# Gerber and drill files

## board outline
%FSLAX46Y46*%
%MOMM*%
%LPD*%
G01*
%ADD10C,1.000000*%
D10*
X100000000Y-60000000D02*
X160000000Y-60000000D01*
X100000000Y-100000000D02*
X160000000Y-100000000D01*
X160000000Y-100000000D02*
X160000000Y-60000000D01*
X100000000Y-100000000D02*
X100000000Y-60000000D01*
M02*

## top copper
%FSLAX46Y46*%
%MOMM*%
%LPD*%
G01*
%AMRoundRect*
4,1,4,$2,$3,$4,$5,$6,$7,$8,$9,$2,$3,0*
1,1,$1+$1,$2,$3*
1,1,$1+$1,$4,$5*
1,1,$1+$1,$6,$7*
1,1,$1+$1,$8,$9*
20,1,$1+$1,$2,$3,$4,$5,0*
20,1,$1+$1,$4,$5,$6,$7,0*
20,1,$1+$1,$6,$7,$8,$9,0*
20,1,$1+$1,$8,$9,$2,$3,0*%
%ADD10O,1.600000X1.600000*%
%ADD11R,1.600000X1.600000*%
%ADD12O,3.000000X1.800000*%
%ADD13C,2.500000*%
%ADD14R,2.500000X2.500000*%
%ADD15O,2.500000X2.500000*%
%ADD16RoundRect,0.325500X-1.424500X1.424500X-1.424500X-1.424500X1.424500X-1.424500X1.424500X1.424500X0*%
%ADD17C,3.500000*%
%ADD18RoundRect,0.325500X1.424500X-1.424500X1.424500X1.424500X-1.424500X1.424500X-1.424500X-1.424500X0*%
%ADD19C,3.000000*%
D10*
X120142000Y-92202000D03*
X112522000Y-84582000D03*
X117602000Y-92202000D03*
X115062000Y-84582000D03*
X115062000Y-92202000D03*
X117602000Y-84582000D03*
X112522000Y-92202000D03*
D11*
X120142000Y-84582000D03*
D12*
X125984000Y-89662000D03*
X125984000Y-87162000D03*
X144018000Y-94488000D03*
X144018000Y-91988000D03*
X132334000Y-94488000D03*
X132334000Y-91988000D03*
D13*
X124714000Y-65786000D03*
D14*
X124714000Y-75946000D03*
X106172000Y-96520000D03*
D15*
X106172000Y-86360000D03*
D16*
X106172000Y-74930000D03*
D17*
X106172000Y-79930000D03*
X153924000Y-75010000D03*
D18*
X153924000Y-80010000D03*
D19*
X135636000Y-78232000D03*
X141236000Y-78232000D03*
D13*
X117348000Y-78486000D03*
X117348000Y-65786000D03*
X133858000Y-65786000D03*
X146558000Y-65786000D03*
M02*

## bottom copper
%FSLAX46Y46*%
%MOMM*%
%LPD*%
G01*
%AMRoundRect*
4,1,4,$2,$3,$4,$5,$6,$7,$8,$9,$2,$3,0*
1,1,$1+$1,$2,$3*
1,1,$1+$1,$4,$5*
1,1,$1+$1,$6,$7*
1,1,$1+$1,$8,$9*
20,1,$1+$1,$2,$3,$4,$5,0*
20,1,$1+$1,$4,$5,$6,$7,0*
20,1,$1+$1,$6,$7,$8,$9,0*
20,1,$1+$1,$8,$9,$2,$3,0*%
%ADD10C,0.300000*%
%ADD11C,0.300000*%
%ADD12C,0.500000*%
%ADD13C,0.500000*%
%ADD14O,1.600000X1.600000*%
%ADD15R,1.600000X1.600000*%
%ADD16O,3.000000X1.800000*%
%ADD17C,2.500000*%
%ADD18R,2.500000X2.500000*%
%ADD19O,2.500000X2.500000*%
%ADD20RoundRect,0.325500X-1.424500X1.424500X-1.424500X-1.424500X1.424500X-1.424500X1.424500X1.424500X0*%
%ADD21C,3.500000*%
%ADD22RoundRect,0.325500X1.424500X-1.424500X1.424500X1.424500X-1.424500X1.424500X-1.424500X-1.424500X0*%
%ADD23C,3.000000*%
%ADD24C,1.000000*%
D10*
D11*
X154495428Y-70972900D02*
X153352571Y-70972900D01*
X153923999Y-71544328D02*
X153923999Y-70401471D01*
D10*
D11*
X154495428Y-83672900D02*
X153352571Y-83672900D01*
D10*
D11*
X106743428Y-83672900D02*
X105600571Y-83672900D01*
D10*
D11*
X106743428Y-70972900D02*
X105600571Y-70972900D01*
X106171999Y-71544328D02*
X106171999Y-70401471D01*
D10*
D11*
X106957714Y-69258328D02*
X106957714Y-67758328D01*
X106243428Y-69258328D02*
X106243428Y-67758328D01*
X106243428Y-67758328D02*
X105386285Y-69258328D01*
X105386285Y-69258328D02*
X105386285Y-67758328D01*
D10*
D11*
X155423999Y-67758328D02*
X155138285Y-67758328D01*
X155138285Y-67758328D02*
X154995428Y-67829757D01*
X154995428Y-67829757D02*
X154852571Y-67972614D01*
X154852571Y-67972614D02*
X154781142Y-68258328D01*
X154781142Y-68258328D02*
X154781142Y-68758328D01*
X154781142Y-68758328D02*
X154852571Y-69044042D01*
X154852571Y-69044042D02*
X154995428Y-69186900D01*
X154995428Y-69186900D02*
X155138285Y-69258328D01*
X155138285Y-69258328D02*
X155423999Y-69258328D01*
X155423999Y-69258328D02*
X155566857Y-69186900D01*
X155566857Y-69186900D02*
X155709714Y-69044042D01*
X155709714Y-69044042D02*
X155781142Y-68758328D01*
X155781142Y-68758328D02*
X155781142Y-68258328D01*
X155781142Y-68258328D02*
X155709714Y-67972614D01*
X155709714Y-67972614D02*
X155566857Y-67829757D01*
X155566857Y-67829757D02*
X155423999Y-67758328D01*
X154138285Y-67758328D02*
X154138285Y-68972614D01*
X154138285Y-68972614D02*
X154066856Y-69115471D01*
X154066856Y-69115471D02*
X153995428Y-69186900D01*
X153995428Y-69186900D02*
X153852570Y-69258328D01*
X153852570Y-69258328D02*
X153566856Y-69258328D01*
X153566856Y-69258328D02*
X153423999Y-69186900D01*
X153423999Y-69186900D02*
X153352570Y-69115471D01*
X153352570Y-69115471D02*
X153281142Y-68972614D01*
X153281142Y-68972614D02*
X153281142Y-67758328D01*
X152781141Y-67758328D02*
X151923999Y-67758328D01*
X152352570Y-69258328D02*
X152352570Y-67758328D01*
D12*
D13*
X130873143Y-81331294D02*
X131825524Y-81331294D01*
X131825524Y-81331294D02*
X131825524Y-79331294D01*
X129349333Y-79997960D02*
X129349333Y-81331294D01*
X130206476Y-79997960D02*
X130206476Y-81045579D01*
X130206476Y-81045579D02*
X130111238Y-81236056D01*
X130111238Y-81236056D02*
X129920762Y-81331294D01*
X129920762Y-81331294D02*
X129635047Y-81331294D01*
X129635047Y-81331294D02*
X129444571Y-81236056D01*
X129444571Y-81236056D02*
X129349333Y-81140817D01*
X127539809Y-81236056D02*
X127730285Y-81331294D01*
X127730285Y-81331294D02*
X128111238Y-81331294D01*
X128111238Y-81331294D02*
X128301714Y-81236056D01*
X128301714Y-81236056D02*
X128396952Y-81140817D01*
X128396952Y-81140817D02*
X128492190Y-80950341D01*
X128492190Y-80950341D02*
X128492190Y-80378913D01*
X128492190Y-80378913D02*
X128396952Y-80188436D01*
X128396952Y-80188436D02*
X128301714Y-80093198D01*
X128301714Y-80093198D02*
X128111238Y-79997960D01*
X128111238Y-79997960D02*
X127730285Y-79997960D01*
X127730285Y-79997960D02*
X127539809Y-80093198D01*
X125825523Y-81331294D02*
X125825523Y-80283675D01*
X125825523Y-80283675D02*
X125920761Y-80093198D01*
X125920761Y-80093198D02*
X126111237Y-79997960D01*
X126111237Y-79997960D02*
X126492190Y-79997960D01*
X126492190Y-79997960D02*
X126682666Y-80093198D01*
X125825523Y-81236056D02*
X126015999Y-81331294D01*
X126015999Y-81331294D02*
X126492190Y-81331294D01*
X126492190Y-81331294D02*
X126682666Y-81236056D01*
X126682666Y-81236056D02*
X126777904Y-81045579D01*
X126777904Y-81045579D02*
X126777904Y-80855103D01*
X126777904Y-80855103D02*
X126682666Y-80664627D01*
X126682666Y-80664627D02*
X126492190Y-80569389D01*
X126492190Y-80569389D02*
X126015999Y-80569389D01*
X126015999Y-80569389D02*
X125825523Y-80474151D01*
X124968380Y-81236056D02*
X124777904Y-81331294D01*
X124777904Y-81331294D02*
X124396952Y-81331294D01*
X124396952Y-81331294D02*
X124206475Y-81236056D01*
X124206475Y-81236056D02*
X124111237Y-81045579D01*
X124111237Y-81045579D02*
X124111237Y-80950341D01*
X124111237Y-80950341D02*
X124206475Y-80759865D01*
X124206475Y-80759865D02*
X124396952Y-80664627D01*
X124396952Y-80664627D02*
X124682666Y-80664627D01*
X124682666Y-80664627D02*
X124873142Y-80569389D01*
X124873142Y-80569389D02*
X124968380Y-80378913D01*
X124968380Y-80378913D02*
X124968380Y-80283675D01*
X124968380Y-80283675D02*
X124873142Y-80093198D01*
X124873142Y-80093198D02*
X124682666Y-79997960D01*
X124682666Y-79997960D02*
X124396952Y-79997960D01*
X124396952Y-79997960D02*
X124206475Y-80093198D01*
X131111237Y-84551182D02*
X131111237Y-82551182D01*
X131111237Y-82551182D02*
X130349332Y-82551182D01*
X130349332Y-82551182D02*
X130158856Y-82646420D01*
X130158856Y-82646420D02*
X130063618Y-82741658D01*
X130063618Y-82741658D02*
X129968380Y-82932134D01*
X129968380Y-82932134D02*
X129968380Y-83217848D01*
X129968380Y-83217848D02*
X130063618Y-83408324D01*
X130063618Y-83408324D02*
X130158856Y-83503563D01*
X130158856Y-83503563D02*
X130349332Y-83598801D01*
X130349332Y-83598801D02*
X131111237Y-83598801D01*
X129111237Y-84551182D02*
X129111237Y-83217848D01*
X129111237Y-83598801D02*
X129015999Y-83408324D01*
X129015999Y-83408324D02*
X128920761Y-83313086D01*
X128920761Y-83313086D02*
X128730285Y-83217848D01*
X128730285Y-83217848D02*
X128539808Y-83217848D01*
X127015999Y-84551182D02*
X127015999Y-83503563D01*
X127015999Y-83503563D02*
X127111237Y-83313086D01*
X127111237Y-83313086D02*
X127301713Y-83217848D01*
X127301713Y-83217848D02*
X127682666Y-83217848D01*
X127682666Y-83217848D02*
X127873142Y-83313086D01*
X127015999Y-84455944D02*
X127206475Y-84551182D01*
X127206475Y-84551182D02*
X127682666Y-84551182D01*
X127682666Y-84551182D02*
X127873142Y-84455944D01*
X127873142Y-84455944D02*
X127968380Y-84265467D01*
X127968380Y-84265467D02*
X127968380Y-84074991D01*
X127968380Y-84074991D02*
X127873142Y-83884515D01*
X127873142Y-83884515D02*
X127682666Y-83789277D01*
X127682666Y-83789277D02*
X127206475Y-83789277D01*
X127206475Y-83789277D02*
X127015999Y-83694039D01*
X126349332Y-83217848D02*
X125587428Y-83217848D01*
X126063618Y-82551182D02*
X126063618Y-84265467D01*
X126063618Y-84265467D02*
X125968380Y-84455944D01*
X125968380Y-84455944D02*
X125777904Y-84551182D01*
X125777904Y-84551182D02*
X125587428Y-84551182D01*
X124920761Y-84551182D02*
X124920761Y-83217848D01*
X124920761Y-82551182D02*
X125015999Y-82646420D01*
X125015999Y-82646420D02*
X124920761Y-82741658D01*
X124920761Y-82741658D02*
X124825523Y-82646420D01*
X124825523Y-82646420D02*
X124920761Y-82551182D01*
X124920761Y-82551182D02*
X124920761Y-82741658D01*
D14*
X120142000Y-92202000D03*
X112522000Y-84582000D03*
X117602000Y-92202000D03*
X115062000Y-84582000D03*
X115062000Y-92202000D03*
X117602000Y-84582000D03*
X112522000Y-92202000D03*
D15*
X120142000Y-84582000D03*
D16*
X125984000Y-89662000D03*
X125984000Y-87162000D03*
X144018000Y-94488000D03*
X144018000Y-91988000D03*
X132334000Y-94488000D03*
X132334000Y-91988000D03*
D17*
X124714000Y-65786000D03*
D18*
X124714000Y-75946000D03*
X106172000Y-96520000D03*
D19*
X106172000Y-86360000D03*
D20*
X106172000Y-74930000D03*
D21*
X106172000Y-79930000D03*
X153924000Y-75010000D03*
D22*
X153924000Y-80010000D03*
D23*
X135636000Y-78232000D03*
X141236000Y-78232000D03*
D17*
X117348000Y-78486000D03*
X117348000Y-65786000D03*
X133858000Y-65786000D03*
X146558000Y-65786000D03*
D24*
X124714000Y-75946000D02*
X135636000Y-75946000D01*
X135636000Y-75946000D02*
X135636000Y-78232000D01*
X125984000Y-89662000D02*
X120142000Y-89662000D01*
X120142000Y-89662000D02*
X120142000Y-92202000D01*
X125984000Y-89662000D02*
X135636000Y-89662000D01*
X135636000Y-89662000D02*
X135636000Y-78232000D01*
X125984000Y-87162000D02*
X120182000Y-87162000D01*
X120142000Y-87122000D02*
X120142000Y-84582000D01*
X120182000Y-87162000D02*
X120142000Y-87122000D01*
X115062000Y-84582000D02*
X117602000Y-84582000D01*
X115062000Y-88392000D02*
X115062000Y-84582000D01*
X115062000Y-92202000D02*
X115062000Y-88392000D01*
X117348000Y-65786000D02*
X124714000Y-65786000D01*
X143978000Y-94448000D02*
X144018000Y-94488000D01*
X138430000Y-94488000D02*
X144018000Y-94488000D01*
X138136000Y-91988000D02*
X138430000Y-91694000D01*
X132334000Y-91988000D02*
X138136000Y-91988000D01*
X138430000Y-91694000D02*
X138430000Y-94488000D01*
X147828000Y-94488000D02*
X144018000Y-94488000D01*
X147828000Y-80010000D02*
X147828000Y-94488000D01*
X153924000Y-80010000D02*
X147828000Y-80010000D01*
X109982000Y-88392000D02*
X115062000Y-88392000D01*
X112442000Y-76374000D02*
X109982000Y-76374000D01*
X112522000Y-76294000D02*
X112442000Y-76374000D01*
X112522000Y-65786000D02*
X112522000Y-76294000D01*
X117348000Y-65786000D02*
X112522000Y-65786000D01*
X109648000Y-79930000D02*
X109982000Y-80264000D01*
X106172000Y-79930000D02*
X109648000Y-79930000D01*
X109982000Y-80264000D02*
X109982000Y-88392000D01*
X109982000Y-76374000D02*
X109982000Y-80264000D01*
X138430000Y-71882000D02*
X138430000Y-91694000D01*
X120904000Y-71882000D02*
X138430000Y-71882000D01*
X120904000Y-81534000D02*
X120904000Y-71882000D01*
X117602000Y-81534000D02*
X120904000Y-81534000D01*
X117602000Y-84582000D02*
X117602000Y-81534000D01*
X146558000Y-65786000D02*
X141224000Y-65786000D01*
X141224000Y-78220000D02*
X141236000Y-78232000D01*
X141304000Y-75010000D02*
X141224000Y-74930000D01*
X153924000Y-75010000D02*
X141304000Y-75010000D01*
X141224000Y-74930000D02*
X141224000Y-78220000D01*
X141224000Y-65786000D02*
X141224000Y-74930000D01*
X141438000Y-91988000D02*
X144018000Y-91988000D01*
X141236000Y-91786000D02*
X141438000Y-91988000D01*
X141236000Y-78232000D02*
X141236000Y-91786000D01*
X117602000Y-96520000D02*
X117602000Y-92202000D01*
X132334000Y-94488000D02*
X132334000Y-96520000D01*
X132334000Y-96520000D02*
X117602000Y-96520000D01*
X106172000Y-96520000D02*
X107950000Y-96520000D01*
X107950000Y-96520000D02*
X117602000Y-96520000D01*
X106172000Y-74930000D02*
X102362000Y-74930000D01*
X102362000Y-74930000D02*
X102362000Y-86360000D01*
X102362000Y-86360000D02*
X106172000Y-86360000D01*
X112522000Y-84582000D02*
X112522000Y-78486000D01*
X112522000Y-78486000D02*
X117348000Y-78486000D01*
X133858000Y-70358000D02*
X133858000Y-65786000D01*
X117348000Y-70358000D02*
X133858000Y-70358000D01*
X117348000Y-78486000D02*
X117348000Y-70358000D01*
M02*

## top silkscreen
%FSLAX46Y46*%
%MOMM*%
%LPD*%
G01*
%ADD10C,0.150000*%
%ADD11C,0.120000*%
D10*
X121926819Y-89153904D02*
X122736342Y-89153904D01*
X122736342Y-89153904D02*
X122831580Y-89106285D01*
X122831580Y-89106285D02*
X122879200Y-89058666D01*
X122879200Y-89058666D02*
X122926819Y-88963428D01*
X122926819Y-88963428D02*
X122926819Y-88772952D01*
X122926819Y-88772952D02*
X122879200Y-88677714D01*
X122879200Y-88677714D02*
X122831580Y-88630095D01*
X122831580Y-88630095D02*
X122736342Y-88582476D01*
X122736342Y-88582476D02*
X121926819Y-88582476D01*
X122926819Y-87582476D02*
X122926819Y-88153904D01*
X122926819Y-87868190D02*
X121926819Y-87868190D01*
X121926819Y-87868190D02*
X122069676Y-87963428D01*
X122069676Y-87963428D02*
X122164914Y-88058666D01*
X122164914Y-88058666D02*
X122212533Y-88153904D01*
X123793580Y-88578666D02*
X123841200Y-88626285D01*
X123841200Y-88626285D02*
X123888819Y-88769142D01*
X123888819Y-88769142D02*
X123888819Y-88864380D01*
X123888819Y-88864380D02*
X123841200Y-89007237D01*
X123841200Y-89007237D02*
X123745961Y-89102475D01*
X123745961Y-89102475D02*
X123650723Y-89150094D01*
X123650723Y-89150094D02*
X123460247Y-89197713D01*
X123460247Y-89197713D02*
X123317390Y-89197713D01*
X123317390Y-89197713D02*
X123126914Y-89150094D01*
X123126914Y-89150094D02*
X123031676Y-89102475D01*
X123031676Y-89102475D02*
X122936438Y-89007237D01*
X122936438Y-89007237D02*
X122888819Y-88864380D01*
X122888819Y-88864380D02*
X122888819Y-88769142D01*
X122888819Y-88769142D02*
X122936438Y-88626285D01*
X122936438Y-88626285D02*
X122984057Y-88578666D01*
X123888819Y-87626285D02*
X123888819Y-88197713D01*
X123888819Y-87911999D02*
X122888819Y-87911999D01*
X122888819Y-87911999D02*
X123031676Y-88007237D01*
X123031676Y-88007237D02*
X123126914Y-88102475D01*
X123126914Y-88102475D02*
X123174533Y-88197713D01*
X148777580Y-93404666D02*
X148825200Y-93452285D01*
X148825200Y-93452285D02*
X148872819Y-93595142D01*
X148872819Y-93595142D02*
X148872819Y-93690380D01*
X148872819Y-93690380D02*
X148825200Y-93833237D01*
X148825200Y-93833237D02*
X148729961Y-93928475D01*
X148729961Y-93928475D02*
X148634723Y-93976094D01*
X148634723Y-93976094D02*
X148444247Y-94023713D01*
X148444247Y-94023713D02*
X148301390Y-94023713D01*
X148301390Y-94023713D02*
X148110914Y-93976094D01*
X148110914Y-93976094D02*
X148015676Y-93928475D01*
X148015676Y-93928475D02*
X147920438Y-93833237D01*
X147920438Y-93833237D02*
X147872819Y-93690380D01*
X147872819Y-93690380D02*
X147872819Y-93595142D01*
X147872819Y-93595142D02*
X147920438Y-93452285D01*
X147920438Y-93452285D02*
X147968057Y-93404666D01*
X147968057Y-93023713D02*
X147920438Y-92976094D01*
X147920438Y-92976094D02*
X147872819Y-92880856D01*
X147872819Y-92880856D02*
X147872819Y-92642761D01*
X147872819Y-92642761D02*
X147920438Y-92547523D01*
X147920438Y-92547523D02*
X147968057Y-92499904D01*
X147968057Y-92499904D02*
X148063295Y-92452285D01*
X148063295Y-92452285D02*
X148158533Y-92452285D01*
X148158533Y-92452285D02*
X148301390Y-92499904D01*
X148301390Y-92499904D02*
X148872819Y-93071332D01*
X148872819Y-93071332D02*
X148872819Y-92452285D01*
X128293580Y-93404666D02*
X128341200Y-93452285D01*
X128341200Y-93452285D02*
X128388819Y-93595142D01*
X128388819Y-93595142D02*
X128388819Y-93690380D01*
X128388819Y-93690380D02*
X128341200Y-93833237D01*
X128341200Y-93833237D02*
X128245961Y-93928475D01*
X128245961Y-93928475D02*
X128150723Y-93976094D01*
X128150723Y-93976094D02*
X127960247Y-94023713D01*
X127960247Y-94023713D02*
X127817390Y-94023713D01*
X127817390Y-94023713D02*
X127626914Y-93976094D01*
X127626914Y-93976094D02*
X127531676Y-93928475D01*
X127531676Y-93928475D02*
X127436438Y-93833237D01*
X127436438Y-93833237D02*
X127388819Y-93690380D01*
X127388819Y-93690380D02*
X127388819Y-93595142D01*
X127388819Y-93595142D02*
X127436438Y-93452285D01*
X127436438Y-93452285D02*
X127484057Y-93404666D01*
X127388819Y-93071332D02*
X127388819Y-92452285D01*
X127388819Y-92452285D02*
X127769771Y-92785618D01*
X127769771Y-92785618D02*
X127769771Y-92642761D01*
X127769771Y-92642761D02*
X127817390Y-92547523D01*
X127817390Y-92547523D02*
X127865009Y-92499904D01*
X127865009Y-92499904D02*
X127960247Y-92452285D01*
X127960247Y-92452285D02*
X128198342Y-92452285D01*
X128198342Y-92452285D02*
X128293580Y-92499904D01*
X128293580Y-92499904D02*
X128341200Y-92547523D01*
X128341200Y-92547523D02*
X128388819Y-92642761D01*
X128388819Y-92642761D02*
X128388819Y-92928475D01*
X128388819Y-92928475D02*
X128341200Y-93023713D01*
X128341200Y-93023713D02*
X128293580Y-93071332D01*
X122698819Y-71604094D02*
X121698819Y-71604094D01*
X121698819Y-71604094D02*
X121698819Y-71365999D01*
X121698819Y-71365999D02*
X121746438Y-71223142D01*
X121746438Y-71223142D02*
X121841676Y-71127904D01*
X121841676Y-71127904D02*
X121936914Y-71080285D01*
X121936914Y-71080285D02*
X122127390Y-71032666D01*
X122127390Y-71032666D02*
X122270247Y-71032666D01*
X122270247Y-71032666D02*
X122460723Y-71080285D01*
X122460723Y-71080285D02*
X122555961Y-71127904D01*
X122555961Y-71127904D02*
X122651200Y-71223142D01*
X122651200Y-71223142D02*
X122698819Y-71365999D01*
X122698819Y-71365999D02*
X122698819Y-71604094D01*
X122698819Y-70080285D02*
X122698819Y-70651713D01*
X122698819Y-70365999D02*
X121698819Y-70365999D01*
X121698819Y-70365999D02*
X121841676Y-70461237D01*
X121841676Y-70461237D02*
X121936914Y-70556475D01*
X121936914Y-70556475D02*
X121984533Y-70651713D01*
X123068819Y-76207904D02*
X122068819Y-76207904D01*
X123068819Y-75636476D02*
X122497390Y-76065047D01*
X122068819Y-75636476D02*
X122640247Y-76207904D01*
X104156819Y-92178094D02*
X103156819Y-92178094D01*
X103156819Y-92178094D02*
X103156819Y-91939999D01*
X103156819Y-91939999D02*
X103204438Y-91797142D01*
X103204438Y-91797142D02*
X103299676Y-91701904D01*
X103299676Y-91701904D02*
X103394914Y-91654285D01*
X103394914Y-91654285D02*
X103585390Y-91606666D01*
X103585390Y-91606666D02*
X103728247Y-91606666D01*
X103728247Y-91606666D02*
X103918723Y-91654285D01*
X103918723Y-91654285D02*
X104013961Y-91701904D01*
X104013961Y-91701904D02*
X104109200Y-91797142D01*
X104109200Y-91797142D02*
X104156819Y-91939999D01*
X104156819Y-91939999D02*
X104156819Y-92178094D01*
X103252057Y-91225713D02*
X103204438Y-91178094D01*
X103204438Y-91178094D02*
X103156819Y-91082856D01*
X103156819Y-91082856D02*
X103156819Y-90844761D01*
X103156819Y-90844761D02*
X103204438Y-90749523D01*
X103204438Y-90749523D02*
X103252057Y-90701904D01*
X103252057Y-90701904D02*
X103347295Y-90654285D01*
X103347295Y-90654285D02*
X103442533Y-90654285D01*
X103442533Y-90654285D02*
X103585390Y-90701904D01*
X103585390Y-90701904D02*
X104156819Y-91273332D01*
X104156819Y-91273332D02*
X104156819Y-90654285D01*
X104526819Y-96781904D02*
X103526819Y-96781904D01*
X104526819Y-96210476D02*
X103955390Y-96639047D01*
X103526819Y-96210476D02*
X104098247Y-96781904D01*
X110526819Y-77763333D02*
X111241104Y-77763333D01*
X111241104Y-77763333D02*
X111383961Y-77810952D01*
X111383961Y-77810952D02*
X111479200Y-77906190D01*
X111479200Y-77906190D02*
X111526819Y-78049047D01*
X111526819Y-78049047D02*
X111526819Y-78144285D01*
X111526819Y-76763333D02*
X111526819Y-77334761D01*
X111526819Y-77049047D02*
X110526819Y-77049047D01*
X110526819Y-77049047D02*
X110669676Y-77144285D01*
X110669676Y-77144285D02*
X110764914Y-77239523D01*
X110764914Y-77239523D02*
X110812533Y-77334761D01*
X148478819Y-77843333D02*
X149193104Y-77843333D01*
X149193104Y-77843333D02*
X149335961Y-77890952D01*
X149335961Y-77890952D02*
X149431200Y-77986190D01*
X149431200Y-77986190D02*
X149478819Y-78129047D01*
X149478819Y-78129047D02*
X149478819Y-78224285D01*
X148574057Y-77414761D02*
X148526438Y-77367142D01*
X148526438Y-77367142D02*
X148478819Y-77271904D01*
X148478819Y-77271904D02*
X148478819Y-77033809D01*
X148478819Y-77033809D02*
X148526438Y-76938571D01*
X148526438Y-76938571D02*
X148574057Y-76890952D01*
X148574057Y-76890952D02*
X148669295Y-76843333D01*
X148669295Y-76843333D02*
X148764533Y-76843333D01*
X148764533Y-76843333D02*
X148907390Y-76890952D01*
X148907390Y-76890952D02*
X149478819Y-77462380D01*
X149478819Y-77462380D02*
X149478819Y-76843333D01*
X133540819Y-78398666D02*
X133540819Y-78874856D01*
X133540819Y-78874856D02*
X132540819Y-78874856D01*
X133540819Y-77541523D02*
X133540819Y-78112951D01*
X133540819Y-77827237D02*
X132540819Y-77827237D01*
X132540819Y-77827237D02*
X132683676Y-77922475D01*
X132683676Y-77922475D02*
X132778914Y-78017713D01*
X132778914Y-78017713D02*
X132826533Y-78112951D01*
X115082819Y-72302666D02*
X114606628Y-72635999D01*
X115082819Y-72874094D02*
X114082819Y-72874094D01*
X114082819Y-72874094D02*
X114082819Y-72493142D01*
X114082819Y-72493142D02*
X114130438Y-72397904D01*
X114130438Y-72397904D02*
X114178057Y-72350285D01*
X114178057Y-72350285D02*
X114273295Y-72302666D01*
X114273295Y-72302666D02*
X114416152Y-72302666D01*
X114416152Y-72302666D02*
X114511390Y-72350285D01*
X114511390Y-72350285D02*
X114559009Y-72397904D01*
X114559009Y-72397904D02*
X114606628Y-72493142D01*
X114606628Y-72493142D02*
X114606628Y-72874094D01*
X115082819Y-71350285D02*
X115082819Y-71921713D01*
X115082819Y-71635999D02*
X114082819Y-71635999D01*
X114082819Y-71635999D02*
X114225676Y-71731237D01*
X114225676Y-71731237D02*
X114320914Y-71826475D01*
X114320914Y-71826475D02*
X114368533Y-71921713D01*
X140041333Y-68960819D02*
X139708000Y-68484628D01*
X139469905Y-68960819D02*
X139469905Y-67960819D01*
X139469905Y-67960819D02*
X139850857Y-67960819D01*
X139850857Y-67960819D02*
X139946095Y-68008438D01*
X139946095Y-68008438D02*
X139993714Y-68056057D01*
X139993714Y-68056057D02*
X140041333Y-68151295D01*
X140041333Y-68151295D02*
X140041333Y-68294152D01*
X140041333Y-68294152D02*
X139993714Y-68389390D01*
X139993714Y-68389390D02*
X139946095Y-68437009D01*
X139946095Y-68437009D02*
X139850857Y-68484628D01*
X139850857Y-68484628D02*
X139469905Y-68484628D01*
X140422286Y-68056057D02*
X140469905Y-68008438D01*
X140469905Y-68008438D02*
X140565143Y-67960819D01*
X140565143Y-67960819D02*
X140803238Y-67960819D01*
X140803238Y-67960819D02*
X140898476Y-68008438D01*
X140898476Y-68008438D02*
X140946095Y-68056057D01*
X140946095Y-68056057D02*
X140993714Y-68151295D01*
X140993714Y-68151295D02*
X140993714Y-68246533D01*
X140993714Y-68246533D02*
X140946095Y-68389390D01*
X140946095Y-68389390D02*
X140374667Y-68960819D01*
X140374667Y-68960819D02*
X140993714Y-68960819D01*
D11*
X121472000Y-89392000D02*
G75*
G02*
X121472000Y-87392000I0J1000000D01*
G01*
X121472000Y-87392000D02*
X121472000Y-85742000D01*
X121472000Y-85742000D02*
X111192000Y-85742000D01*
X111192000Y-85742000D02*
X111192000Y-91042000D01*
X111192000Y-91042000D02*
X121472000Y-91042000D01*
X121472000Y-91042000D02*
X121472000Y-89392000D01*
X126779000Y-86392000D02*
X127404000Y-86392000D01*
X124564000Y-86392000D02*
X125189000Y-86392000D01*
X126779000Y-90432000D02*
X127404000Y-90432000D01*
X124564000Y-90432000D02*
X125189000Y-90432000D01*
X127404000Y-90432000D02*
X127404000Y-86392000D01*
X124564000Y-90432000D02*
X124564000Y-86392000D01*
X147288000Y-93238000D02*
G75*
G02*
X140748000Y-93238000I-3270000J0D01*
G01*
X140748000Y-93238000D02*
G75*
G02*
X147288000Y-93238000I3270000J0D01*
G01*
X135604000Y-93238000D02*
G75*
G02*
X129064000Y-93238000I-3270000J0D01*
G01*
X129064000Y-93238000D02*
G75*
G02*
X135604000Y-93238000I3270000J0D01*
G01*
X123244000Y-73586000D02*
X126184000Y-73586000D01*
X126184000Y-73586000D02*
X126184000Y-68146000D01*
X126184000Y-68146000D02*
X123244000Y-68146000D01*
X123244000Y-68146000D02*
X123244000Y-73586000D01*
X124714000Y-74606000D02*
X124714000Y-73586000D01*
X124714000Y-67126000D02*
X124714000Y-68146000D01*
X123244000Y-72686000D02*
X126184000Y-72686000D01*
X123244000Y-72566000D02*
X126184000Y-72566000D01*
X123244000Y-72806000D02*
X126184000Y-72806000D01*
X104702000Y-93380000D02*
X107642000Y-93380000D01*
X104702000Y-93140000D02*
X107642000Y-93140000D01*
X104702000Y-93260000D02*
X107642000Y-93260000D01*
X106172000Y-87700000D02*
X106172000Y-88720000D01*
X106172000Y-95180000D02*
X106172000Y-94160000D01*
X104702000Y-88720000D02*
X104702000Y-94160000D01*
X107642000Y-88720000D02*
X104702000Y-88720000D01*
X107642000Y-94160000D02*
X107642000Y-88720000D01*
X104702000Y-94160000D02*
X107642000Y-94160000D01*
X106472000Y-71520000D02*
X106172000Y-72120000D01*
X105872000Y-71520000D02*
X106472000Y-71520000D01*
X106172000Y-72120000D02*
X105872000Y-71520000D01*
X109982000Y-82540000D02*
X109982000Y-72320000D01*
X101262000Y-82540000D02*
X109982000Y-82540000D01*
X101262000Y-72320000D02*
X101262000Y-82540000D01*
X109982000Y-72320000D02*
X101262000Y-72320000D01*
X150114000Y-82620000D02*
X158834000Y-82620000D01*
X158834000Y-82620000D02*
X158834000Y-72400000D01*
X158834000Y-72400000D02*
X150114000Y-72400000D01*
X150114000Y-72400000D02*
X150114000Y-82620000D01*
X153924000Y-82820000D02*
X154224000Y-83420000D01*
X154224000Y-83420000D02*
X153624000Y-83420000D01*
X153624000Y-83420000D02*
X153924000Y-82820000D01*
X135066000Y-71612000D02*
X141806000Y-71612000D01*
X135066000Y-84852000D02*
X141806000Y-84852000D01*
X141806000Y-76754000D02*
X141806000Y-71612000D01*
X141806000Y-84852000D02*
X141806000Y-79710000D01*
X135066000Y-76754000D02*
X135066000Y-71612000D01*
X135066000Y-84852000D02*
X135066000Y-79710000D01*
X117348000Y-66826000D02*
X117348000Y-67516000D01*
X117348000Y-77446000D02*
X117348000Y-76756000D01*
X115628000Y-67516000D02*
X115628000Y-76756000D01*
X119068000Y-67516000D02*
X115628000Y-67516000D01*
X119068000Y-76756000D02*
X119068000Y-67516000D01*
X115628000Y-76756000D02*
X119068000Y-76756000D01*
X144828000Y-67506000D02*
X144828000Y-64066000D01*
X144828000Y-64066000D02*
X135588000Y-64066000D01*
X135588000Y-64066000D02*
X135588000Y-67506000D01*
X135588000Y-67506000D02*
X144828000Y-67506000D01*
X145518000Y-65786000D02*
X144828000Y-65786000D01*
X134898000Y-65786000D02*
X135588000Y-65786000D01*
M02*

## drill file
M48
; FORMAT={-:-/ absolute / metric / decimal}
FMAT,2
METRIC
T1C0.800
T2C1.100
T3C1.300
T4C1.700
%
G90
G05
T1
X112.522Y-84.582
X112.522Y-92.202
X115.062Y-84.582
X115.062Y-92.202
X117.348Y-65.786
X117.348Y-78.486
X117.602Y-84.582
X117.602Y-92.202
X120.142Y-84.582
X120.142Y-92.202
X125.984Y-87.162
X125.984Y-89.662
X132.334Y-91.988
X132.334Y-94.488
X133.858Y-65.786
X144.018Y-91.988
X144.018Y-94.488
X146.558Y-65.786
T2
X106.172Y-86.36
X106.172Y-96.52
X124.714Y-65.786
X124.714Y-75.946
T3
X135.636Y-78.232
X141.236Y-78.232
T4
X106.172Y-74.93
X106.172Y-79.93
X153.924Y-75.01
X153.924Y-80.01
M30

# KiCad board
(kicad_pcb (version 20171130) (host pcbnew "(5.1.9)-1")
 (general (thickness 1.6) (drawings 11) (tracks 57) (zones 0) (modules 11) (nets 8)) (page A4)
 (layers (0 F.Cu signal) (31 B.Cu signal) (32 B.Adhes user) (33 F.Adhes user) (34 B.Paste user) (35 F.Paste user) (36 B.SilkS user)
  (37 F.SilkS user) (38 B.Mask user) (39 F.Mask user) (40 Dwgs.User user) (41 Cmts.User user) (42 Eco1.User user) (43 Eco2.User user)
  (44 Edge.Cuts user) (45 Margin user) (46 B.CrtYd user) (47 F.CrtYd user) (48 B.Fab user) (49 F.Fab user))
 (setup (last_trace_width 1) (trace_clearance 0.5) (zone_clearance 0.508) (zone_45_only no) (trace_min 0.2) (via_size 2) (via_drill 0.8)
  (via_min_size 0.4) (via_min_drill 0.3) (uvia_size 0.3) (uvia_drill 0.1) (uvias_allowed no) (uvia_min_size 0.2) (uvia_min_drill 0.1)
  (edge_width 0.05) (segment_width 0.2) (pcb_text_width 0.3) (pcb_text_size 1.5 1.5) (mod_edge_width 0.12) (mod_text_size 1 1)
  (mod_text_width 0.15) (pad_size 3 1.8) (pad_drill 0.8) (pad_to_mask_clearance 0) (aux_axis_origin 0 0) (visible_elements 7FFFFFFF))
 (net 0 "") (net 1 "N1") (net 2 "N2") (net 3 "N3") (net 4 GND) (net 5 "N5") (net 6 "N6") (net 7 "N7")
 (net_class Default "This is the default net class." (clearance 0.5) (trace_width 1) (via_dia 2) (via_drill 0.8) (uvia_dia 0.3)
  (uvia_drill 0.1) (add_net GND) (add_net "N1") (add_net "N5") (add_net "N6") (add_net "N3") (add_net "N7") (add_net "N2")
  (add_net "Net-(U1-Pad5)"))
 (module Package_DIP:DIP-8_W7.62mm (layer F.Cu) (at 120.142 84.582 270)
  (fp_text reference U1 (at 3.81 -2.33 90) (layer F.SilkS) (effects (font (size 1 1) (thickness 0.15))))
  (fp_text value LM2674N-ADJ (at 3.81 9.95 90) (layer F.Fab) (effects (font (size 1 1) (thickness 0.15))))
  (fp_arc (start 3.81 -1.33) (end 2.81 -1.33) (angle -180) (layer F.SilkS) (width 0.12))
  (fp_line (start 2.81 -1.33) (end 1.16 -1.33) (layer F.SilkS) (width 0.12))
  (fp_line (start 1.16 -1.33) (end 1.16 8.95) (layer F.SilkS) (width 0.12))
  (fp_line (start 1.16 8.95) (end 6.46 8.95) (layer F.SilkS) (width 0.12))
  (fp_line (start 6.46 8.95) (end 6.46 -1.33) (layer F.SilkS) (width 0.12))
  (fp_line (start 6.46 -1.33) (end 4.81 -1.33) (layer F.SilkS) (width 0.12))
  (pad 8 thru_hole oval (at 7.62 0 270) (size 1.6 1.6) (drill 0.8) (layers *.Cu *.Mask) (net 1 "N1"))
  (pad 4 thru_hole oval (at 0 7.62 270) (size 1.6 1.6) (drill 0.8) (layers *.Cu *.Mask) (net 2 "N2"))
  (pad 7 thru_hole oval (at 7.62 2.54 270) (size 1.6 1.6) (drill 0.8) (layers *.Cu *.Mask) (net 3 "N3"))
  (pad 3 thru_hole oval (at 0 5.08 270) (size 1.6 1.6) (drill 0.8) (layers *.Cu *.Mask) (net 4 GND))
  (pad 6 thru_hole oval (at 7.62 5.08 270) (size 1.6 1.6) (drill 0.8) (layers *.Cu *.Mask) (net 4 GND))
  (pad 2 thru_hole oval (at 0 2.54 270) (size 1.6 1.6) (drill 0.8) (layers *.Cu *.Mask) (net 4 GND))
  (pad 5 thru_hole oval (at 7.62 7.62 270) (size 1.6 1.6) (drill 0.8) (layers *.Cu *.Mask))
  (pad 1 thru_hole rect (at 0 0 270) (size 1.6 1.6) (drill 0.8) (layers *.Cu *.Mask) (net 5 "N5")))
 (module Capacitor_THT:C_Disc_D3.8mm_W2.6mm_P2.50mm (layer F.Cu) (at 125.984 89.662 90)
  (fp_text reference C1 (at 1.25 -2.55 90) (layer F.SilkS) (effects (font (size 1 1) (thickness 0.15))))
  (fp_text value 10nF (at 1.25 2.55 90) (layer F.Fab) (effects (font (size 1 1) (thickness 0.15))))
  (fp_line (start 3.27 0.795) (end 3.27 1.42) (layer F.SilkS) (width 0.12))
  (fp_line (start 3.27 -1.42) (end 3.27 -0.795) (layer F.SilkS) (width 0.12))
  (fp_line (start -0.77 0.795) (end -0.77 1.42) (layer F.SilkS) (width 0.12))
  (fp_line (start -0.77 -1.42) (end -0.77 -0.795) (layer F.SilkS) (width 0.12))
  (fp_line (start -0.77 1.42) (end 3.27 1.42) (layer F.SilkS) (width 0.12))
  (fp_line (start -0.77 -1.42) (end 3.27 -1.42) (layer F.SilkS) (width 0.12))
  (pad 1 thru_hole oval (at 0 0 90) (size 1.8 3) (drill 0.8) (layers *.Cu *.Mask) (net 1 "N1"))
  (pad 2 thru_hole oval (at 2.5 0 90) (size 1.8 3) (drill 0.8) (layers *.Cu *.Mask) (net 5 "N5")))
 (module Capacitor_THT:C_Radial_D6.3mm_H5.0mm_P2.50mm (layer F.Cu) (at 144.018 91.988 270)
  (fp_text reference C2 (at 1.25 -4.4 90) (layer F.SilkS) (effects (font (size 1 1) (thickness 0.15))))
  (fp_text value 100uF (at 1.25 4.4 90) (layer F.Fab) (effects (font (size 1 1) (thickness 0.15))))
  (fp_circle (center 1.25 0) (end 4.52 0) (layer F.SilkS) (width 0.12))
  (pad 2 thru_hole oval (at 2.5 0 270) (size 1.8 3) (drill 0.8) (layers *.Cu *.Mask) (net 4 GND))
  (pad 1 thru_hole oval (at 0 0 270) (size 1.8 3) (drill 0.8) (layers *.Cu *.Mask) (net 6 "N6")))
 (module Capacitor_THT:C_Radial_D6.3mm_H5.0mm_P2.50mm (layer F.Cu) (at 132.334 94.488 90)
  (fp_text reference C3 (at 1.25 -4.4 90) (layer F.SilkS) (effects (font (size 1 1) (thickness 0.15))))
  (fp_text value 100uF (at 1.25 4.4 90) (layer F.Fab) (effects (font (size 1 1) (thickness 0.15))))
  (fp_circle (center 1.25 0) (end 4.52 0) (layer F.SilkS) (width 0.12))
  (pad 1 thru_hole oval (at 0 0 90) (size 1.8 3) (drill 0.8) (layers *.Cu *.Mask) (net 3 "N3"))
  (pad 2 thru_hole oval (at 2.5 0 90) (size 1.8 3) (drill 0.8) (layers *.Cu *.Mask) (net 4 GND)))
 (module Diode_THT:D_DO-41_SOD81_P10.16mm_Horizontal (layer F.Cu) (at 124.714 75.946 90)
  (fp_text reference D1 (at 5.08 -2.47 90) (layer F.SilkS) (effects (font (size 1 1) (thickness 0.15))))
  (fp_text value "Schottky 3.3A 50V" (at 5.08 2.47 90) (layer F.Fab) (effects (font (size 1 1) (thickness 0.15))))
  (fp_line (start 2.36 -1.47) (end 2.36 1.47) (layer F.SilkS) (width 0.12))
  (fp_line (start 2.36 1.47) (end 7.8 1.47) (layer F.SilkS) (width 0.12))
  (fp_line (start 7.8 1.47) (end 7.8 -1.47) (layer F.SilkS) (width 0.12))
  (fp_line (start 7.8 -1.47) (end 2.36 -1.47) (layer F.SilkS) (width 0.12))
  (fp_line (start 1.34 0) (end 2.36 0) (layer F.SilkS) (width 0.12))
  (fp_line (start 8.82 0) (end 7.8 0) (layer F.SilkS) (width 0.12))
  (fp_line (start 3.26 -1.47) (end 3.26 1.47) (layer F.SilkS) (width 0.12))
  (fp_line (start 3.38 -1.47) (end 3.38 1.47) (layer F.SilkS) (width 0.12))
  (fp_line (start 3.14 -1.47) (end 3.14 1.47) (layer F.SilkS) (width 0.12))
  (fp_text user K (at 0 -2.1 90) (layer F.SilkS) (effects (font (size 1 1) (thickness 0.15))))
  (pad 2 thru_hole circle (at 10.16 0 90) (size 2.5 2.5) (drill 1.1) (layers *.Cu *.Mask) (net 4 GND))
  (pad 1 thru_hole rect (at 0 0 90) (size 2.5 2.5) (drill 1.1) (layers *.Cu *.Mask) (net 1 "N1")))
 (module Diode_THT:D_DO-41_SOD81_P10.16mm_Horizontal (layer F.Cu) (at 106.172 96.52 90)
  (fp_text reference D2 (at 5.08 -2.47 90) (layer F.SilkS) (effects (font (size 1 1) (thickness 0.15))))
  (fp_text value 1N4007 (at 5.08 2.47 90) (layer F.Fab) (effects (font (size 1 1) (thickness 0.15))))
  (fp_line (start 3.14 -1.47) (end 3.14 1.47) (layer F.SilkS) (width 0.12))
  (fp_line (start 3.38 -1.47) (end 3.38 1.47) (layer F.SilkS) (width 0.12))
  (fp_line (start 3.26 -1.47) (end 3.26 1.47) (layer F.SilkS) (width 0.12))
  (fp_line (start 8.82 0) (end 7.8 0) (layer F.SilkS) (width 0.12))
  (fp_line (start 1.34 0) (end 2.36 0) (layer F.SilkS) (width 0.12))
  (fp_line (start 7.8 -1.47) (end 2.36 -1.47) (layer F.SilkS) (width 0.12))
  (fp_line (start 7.8 1.47) (end 7.8 -1.47) (layer F.SilkS) (width 0.12))
  (fp_line (start 2.36 1.47) (end 7.8 1.47) (layer F.SilkS) (width 0.12))
  (fp_line (start 2.36 -1.47) (end 2.36 1.47) (layer F.SilkS) (width 0.12))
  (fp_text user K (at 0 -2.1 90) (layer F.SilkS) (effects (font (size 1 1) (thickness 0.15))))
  (pad 1 thru_hole rect (at 0 0 90) (size 2.5 2.5) (drill 1.1) (layers *.Cu *.Mask) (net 3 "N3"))
  (pad 2 thru_hole oval (at 10.16 0 90) (size 2.5 2.5) (drill 1.1) (layers *.Cu *.Mask) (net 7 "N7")))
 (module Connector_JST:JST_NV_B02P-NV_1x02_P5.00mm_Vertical (layer F.Cu) (at 106.172 74.93 270)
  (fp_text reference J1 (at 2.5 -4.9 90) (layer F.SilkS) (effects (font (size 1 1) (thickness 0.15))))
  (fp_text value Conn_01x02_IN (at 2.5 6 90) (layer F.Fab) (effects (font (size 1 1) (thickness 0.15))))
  (fp_line (start -3.41 -0.3) (end -2.81 0) (layer F.SilkS) (width 0.12))
  (fp_line (start -3.41 0.3) (end -3.41 -0.3) (layer F.SilkS) (width 0.12))
  (fp_line (start -2.81 0) (end -3.41 0.3) (layer F.SilkS) (width 0.12))
  (fp_line (start 7.61 -3.81) (end -2.61 -3.81) (layer F.SilkS) (width 0.12))
  (fp_line (start 7.61 4.91) (end 7.61 -3.81) (layer F.SilkS) (width 0.12))
  (fp_line (start -2.61 4.91) (end 7.61 4.91) (layer F.SilkS) (width 0.12))
  (fp_line (start -2.61 -3.81) (end -2.61 4.91) (layer F.SilkS) (width 0.12))
  (pad 1 thru_hole roundrect (at 0 0 270) (size 3.5 3.5) (drill 1.7) (layers *.Cu *.Mask) (roundrect_rratio 0.09300000000000001)
   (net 7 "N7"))
  (pad 2 thru_hole circle (at 5 0 270) (size 3.5 3.5) (drill 1.7) (layers *.Cu *.Mask) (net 4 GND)))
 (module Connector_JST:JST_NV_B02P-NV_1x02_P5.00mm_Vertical (layer F.Cu) (at 153.924 80.01 90)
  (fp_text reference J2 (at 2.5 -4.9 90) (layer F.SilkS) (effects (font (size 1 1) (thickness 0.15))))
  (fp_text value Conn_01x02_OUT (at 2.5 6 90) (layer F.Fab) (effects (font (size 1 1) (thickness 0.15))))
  (fp_line (start -2.61 -3.81) (end -2.61 4.91) (layer F.SilkS) (width 0.12))
  (fp_line (start -2.61 4.91) (end 7.61 4.91) (layer F.SilkS) (width 0.12))
  (fp_line (start 7.61 4.91) (end 7.61 -3.81) (layer F.SilkS) (width 0.12))
  (fp_line (start 7.61 -3.81) (end -2.61 -3.81) (layer F.SilkS) (width 0.12))
  (fp_line (start -2.81 0) (end -3.41 0.3) (layer F.SilkS) (width 0.12))
  (fp_line (start -3.41 0.3) (end -3.41 -0.3) (layer F.SilkS) (width 0.12))
  (fp_line (start -3.41 -0.3) (end -2.81 0) (layer F.SilkS) (width 0.12))
  (pad 2 thru_hole circle (at 5 0 90) (size 3.5 3.5) (drill 1.7) (layers *.Cu *.Mask) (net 6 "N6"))
  (pad 1 thru_hole roundrect (at 0 0 90) (size 3.5 3.5) (drill 1.7) (layers *.Cu *.Mask) (roundrect_rratio 0.09300000000000001) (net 4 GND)))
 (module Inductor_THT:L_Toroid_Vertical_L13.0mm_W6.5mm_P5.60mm (layer F.Cu) (at 135.636 78.232 90)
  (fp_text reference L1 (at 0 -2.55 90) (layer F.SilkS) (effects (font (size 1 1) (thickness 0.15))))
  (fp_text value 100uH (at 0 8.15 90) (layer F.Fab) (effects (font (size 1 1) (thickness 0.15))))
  (fp_line (start 6.62 -0.57) (end 6.62 6.17) (layer F.SilkS) (width 0.12))
  (fp_line (start -6.62 -0.57) (end -6.62 6.17) (layer F.SilkS) (width 0.12))
  (fp_line (start 1.478 6.17) (end 6.62 6.17) (layer F.SilkS) (width 0.12))
  (fp_line (start -6.62 6.17) (end -1.478 6.17) (layer F.SilkS) (width 0.12))
  (fp_line (start 1.478 -0.57) (end 6.62 -0.57) (layer F.SilkS) (width 0.12))
  (fp_line (start -6.62 -0.57) (end -1.478 -0.57) (layer F.SilkS) (width 0.12))
  (pad 1 thru_hole circle (at 0 0 90) (size 3 3) (drill 1.3) (layers *.Cu *.Mask) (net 1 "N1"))
  (pad 2 thru_hole circle (at 0 5.6 90) (size 3 3) (drill 1.3) (layers *.Cu *.Mask) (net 6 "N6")))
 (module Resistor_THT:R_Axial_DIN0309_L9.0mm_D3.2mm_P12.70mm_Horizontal (layer F.Cu) (at 117.348 78.486 90)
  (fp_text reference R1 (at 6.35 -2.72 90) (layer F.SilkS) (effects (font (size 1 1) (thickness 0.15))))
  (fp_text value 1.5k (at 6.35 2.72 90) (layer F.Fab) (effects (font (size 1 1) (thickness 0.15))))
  (fp_line (start 11.66 0) (end 10.97 0) (layer F.SilkS) (width 0.12))
  (fp_line (start 1.04 0) (end 1.73 0) (layer F.SilkS) (width 0.12))
  (fp_line (start 10.97 -1.72) (end 1.73 -1.72) (layer F.SilkS) (width 0.12))
  (fp_line (start 10.97 1.72) (end 10.97 -1.72) (layer F.SilkS) (width 0.12))
  (fp_line (start 1.73 1.72) (end 10.97 1.72) (layer F.SilkS) (width 0.12))
  (fp_line (start 1.73 -1.72) (end 1.73 1.72) (layer F.SilkS) (width 0.12))
  (pad 1 thru_hole circle (at 0 0 90) (size 2.5 2.5) (drill 0.8) (layers *.Cu *.Mask) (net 2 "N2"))
  (pad 2 thru_hole circle (at 12.7 0 90) (size 2.5 2.5) (drill 0.8) (layers *.Cu *.Mask) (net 4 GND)))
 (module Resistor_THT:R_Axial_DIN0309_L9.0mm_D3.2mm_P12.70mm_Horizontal (layer F.Cu) (at 146.558 65.786 180)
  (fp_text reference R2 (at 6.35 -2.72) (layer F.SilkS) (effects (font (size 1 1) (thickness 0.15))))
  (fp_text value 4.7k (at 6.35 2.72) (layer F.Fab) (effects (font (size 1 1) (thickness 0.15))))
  (fp_line (start 1.73 -1.72) (end 1.73 1.72) (layer F.SilkS) (width 0.12))
  (fp_line (start 1.73 1.72) (end 10.97 1.72) (layer F.SilkS) (width 0.12))
  (fp_line (start 10.97 1.72) (end 10.97 -1.72) (layer F.SilkS) (width 0.12))
  (fp_line (start 10.97 -1.72) (end 1.73 -1.72) (layer F.SilkS) (width 0.12))
  (fp_line (start 1.04 0) (end 1.73 0) (layer F.SilkS) (width 0.12))
  (fp_line (start 11.66 0) (end 10.97 0) (layer F.SilkS) (width 0.12))
  (pad 2 thru_hole circle (at 12.7 0 180) (size 2.5 2.5) (drill 0.8) (layers *.Cu *.Mask) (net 2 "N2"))
  (pad 1 thru_hole circle (at 0 0 180) (size 2.5 2.5) (drill 0.8) (layers *.Cu *.Mask) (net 6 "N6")))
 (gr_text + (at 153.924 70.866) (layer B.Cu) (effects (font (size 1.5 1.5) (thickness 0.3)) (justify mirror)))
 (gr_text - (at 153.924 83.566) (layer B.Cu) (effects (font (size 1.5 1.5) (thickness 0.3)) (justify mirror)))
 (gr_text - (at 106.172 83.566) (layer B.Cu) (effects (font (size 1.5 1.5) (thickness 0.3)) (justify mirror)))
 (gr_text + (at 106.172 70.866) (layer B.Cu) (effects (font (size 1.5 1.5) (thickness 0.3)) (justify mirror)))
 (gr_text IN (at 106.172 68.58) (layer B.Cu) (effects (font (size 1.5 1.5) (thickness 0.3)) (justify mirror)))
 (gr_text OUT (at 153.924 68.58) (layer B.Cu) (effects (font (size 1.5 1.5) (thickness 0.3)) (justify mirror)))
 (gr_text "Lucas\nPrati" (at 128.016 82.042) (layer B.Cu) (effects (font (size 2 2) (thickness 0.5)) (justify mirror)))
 (gr_line (start 100 60) (end 160 60) (layer Edge.Cuts) (width 1))
 (gr_line (start 100 100) (end 160 100) (layer Edge.Cuts) (width 1))
 (gr_line (start 160 100) (end 160 60) (layer Edge.Cuts) (width 1))
 (gr_line (start 100 100) (end 100 60) (layer Edge.Cuts) (width 1))
 (segment (start 124.714 75.946) (end 135.636 75.946) (width 1) (layer B.Cu) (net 1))
 (segment (start 135.636 75.946) (end 135.636 78.232) (width 1) (layer B.Cu) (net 1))
 (segment (start 125.984 89.662) (end 120.142 89.662) (width 1) (layer B.Cu) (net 1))
 (segment (start 120.142 89.662) (end 120.142 92.202) (width 1) (layer B.Cu) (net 1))
 (segment (start 125.984 89.662) (end 135.636 89.662) (width 1) (layer B.Cu) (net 1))
 (segment (start 135.636 89.662) (end 135.636 78.232) (width 1) (layer B.Cu) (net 1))
 (segment (start 125.984 87.162) (end 120.182 87.162) (width 1) (layer B.Cu) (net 5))
 (segment (start 120.142 87.122) (end 120.142 84.582) (width 1) (layer B.Cu) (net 5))
 (segment (start 120.182 87.162) (end 120.142 87.122) (width 1) (layer B.Cu) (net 5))
 (segment (start 115.062 84.582) (end 117.602 84.582) (width 1) (layer B.Cu) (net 4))
 (segment (start 115.062 88.392) (end 115.062 84.582) (width 1) (layer B.Cu) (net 4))
 (segment (start 115.062 92.202) (end 115.062 88.392) (width 1) (layer B.Cu) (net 4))
 (segment (start 117.348 65.786) (end 124.714 65.786) (width 1) (layer B.Cu) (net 4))
 (segment (start 143.978 94.448) (end 144.018 94.488) (width 1) (layer B.Cu) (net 4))
 (segment (start 138.43 94.488) (end 144.018 94.488) (width 1) (layer B.Cu) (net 4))
 (segment (start 138.136 91.988) (end 138.43 91.694) (width 1) (layer B.Cu) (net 4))
 (segment (start 132.334 91.988) (end 138.136 91.988) (width 1) (layer B.Cu) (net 4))
 (segment (start 138.43 91.694) (end 138.43 94.488) (width 1) (layer B.Cu) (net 4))
 (segment (start 147.828 94.488) (end 144.018 94.488) (width 1) (layer B.Cu) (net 4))
 (segment (start 147.828 80.01) (end 147.828 94.488) (width 1) (layer B.Cu) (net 4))
 (segment (start 153.924 80.01) (end 147.828 80.01) (width 1) (layer B.Cu) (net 4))
 (segment (start 109.982 88.392) (end 115.062 88.392) (width 1) (layer B.Cu) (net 4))
 (segment (start 112.442 76.374) (end 109.982 76.374) (width 1) (layer B.Cu) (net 4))
 (segment (start 112.522 76.294) (end 112.442 76.374) (width 1) (layer B.Cu) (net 4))
 (segment (start 112.522 65.786) (end 112.522 76.294) (width 1) (layer B.Cu) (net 4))
 (segment (start 117.348 65.786) (end 112.522 65.786) (width 1) (layer B.Cu) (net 4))
 (segment (start 109.648 79.93) (end 109.982 80.264) (width 1) (layer B.Cu) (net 4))
 (segment (start 106.172 79.93) (end 109.648 79.93) (width 1) (layer B.Cu) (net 4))
 (segment (start 109.982 80.264) (end 109.982 88.392) (width 1) (layer B.Cu) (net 4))
 (segment (start 109.982 76.374) (end 109.982 80.264) (width 1) (layer B.Cu) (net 4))
 (segment (start 138.43 71.882) (end 138.43 91.694) (width 1) (layer B.Cu) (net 4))
 (segment (start 120.904 71.882) (end 138.43 71.882) (width 1) (layer B.Cu) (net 4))
 (segment (start 120.904 81.534) (end 120.904 71.882) (width 1) (layer B.Cu) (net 4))
 (segment (start 117.602 81.534) (end 120.904 81.534) (width 1) (layer B.Cu) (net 4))
 (segment (start 117.602 84.582) (end 117.602 81.534) (width 1) (layer B.Cu) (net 4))
 (segment (start 146.558 65.786) (end 141.224 65.786) (width 1) (layer B.Cu) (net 6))
 (segment (start 141.224 78.22) (end 141.236 78.232) (width 1) (layer B.Cu) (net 6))
 (segment (start 141.304 75.01) (end 141.224 74.93) (width 1) (layer B.Cu) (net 6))
 (segment (start 153.924 75.01) (end 141.304 75.01) (width 1) (layer B.Cu) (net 6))
 (segment (start 141.224 74.93) (end 141.224 78.22) (width 1) (layer B.Cu) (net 6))
 (segment (start 141.224 65.786) (end 141.224 74.93) (width 1) (layer B.Cu) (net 6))
 (segment (start 141.438 91.988) (end 144.018 91.988) (width 1) (layer B.Cu) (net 6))
 (segment (start 141.236 91.786) (end 141.438 91.988) (width 1) (layer B.Cu) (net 6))
 (segment (start 141.236 78.232) (end 141.236 91.786) (width 1) (layer B.Cu) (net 6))
 (segment (start 117.602 96.52) (end 117.602 92.202) (width 1) (layer B.Cu) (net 3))
 (segment (start 132.334 94.488) (end 132.334 96.52) (width 1) (layer B.Cu) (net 3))
 (segment (start 132.334 96.52) (end 117.602 96.52) (width 1) (layer B.Cu) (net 3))
 (segment (start 106.172 96.52) (end 107.95 96.52) (width 1) (layer B.Cu) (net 3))
 (segment (start 107.95 96.52) (end 117.602 96.52) (width 1) (layer B.Cu) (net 3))
 (segment (start 106.172 74.93) (end 102.362 74.93) (width 1) (layer B.Cu) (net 7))
 (segment (start 102.362 74.93) (end 102.362 86.36) (width 1) (layer B.Cu) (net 7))
 (segment (start 102.362 86.36) (end 106.172 86.36) (width 1) (layer B.Cu) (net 7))
 (segment (start 112.522 84.582) (end 112.522 78.486) (width 1) (layer B.Cu) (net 2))
 (segment (start 112.522 78.486) (end 117.348 78.486) (width 1) (layer B.Cu) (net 2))
 (segment (start 133.858 70.358) (end 133.858 65.786) (width 1) (layer B.Cu) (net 2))
 (segment (start 117.348 70.358) (end 133.858 70.358) (width 1) (layer B.Cu) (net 2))
 (segment (start 117.348 78.486) (end 117.348 70.358) (width 1) (layer B.Cu) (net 2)))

